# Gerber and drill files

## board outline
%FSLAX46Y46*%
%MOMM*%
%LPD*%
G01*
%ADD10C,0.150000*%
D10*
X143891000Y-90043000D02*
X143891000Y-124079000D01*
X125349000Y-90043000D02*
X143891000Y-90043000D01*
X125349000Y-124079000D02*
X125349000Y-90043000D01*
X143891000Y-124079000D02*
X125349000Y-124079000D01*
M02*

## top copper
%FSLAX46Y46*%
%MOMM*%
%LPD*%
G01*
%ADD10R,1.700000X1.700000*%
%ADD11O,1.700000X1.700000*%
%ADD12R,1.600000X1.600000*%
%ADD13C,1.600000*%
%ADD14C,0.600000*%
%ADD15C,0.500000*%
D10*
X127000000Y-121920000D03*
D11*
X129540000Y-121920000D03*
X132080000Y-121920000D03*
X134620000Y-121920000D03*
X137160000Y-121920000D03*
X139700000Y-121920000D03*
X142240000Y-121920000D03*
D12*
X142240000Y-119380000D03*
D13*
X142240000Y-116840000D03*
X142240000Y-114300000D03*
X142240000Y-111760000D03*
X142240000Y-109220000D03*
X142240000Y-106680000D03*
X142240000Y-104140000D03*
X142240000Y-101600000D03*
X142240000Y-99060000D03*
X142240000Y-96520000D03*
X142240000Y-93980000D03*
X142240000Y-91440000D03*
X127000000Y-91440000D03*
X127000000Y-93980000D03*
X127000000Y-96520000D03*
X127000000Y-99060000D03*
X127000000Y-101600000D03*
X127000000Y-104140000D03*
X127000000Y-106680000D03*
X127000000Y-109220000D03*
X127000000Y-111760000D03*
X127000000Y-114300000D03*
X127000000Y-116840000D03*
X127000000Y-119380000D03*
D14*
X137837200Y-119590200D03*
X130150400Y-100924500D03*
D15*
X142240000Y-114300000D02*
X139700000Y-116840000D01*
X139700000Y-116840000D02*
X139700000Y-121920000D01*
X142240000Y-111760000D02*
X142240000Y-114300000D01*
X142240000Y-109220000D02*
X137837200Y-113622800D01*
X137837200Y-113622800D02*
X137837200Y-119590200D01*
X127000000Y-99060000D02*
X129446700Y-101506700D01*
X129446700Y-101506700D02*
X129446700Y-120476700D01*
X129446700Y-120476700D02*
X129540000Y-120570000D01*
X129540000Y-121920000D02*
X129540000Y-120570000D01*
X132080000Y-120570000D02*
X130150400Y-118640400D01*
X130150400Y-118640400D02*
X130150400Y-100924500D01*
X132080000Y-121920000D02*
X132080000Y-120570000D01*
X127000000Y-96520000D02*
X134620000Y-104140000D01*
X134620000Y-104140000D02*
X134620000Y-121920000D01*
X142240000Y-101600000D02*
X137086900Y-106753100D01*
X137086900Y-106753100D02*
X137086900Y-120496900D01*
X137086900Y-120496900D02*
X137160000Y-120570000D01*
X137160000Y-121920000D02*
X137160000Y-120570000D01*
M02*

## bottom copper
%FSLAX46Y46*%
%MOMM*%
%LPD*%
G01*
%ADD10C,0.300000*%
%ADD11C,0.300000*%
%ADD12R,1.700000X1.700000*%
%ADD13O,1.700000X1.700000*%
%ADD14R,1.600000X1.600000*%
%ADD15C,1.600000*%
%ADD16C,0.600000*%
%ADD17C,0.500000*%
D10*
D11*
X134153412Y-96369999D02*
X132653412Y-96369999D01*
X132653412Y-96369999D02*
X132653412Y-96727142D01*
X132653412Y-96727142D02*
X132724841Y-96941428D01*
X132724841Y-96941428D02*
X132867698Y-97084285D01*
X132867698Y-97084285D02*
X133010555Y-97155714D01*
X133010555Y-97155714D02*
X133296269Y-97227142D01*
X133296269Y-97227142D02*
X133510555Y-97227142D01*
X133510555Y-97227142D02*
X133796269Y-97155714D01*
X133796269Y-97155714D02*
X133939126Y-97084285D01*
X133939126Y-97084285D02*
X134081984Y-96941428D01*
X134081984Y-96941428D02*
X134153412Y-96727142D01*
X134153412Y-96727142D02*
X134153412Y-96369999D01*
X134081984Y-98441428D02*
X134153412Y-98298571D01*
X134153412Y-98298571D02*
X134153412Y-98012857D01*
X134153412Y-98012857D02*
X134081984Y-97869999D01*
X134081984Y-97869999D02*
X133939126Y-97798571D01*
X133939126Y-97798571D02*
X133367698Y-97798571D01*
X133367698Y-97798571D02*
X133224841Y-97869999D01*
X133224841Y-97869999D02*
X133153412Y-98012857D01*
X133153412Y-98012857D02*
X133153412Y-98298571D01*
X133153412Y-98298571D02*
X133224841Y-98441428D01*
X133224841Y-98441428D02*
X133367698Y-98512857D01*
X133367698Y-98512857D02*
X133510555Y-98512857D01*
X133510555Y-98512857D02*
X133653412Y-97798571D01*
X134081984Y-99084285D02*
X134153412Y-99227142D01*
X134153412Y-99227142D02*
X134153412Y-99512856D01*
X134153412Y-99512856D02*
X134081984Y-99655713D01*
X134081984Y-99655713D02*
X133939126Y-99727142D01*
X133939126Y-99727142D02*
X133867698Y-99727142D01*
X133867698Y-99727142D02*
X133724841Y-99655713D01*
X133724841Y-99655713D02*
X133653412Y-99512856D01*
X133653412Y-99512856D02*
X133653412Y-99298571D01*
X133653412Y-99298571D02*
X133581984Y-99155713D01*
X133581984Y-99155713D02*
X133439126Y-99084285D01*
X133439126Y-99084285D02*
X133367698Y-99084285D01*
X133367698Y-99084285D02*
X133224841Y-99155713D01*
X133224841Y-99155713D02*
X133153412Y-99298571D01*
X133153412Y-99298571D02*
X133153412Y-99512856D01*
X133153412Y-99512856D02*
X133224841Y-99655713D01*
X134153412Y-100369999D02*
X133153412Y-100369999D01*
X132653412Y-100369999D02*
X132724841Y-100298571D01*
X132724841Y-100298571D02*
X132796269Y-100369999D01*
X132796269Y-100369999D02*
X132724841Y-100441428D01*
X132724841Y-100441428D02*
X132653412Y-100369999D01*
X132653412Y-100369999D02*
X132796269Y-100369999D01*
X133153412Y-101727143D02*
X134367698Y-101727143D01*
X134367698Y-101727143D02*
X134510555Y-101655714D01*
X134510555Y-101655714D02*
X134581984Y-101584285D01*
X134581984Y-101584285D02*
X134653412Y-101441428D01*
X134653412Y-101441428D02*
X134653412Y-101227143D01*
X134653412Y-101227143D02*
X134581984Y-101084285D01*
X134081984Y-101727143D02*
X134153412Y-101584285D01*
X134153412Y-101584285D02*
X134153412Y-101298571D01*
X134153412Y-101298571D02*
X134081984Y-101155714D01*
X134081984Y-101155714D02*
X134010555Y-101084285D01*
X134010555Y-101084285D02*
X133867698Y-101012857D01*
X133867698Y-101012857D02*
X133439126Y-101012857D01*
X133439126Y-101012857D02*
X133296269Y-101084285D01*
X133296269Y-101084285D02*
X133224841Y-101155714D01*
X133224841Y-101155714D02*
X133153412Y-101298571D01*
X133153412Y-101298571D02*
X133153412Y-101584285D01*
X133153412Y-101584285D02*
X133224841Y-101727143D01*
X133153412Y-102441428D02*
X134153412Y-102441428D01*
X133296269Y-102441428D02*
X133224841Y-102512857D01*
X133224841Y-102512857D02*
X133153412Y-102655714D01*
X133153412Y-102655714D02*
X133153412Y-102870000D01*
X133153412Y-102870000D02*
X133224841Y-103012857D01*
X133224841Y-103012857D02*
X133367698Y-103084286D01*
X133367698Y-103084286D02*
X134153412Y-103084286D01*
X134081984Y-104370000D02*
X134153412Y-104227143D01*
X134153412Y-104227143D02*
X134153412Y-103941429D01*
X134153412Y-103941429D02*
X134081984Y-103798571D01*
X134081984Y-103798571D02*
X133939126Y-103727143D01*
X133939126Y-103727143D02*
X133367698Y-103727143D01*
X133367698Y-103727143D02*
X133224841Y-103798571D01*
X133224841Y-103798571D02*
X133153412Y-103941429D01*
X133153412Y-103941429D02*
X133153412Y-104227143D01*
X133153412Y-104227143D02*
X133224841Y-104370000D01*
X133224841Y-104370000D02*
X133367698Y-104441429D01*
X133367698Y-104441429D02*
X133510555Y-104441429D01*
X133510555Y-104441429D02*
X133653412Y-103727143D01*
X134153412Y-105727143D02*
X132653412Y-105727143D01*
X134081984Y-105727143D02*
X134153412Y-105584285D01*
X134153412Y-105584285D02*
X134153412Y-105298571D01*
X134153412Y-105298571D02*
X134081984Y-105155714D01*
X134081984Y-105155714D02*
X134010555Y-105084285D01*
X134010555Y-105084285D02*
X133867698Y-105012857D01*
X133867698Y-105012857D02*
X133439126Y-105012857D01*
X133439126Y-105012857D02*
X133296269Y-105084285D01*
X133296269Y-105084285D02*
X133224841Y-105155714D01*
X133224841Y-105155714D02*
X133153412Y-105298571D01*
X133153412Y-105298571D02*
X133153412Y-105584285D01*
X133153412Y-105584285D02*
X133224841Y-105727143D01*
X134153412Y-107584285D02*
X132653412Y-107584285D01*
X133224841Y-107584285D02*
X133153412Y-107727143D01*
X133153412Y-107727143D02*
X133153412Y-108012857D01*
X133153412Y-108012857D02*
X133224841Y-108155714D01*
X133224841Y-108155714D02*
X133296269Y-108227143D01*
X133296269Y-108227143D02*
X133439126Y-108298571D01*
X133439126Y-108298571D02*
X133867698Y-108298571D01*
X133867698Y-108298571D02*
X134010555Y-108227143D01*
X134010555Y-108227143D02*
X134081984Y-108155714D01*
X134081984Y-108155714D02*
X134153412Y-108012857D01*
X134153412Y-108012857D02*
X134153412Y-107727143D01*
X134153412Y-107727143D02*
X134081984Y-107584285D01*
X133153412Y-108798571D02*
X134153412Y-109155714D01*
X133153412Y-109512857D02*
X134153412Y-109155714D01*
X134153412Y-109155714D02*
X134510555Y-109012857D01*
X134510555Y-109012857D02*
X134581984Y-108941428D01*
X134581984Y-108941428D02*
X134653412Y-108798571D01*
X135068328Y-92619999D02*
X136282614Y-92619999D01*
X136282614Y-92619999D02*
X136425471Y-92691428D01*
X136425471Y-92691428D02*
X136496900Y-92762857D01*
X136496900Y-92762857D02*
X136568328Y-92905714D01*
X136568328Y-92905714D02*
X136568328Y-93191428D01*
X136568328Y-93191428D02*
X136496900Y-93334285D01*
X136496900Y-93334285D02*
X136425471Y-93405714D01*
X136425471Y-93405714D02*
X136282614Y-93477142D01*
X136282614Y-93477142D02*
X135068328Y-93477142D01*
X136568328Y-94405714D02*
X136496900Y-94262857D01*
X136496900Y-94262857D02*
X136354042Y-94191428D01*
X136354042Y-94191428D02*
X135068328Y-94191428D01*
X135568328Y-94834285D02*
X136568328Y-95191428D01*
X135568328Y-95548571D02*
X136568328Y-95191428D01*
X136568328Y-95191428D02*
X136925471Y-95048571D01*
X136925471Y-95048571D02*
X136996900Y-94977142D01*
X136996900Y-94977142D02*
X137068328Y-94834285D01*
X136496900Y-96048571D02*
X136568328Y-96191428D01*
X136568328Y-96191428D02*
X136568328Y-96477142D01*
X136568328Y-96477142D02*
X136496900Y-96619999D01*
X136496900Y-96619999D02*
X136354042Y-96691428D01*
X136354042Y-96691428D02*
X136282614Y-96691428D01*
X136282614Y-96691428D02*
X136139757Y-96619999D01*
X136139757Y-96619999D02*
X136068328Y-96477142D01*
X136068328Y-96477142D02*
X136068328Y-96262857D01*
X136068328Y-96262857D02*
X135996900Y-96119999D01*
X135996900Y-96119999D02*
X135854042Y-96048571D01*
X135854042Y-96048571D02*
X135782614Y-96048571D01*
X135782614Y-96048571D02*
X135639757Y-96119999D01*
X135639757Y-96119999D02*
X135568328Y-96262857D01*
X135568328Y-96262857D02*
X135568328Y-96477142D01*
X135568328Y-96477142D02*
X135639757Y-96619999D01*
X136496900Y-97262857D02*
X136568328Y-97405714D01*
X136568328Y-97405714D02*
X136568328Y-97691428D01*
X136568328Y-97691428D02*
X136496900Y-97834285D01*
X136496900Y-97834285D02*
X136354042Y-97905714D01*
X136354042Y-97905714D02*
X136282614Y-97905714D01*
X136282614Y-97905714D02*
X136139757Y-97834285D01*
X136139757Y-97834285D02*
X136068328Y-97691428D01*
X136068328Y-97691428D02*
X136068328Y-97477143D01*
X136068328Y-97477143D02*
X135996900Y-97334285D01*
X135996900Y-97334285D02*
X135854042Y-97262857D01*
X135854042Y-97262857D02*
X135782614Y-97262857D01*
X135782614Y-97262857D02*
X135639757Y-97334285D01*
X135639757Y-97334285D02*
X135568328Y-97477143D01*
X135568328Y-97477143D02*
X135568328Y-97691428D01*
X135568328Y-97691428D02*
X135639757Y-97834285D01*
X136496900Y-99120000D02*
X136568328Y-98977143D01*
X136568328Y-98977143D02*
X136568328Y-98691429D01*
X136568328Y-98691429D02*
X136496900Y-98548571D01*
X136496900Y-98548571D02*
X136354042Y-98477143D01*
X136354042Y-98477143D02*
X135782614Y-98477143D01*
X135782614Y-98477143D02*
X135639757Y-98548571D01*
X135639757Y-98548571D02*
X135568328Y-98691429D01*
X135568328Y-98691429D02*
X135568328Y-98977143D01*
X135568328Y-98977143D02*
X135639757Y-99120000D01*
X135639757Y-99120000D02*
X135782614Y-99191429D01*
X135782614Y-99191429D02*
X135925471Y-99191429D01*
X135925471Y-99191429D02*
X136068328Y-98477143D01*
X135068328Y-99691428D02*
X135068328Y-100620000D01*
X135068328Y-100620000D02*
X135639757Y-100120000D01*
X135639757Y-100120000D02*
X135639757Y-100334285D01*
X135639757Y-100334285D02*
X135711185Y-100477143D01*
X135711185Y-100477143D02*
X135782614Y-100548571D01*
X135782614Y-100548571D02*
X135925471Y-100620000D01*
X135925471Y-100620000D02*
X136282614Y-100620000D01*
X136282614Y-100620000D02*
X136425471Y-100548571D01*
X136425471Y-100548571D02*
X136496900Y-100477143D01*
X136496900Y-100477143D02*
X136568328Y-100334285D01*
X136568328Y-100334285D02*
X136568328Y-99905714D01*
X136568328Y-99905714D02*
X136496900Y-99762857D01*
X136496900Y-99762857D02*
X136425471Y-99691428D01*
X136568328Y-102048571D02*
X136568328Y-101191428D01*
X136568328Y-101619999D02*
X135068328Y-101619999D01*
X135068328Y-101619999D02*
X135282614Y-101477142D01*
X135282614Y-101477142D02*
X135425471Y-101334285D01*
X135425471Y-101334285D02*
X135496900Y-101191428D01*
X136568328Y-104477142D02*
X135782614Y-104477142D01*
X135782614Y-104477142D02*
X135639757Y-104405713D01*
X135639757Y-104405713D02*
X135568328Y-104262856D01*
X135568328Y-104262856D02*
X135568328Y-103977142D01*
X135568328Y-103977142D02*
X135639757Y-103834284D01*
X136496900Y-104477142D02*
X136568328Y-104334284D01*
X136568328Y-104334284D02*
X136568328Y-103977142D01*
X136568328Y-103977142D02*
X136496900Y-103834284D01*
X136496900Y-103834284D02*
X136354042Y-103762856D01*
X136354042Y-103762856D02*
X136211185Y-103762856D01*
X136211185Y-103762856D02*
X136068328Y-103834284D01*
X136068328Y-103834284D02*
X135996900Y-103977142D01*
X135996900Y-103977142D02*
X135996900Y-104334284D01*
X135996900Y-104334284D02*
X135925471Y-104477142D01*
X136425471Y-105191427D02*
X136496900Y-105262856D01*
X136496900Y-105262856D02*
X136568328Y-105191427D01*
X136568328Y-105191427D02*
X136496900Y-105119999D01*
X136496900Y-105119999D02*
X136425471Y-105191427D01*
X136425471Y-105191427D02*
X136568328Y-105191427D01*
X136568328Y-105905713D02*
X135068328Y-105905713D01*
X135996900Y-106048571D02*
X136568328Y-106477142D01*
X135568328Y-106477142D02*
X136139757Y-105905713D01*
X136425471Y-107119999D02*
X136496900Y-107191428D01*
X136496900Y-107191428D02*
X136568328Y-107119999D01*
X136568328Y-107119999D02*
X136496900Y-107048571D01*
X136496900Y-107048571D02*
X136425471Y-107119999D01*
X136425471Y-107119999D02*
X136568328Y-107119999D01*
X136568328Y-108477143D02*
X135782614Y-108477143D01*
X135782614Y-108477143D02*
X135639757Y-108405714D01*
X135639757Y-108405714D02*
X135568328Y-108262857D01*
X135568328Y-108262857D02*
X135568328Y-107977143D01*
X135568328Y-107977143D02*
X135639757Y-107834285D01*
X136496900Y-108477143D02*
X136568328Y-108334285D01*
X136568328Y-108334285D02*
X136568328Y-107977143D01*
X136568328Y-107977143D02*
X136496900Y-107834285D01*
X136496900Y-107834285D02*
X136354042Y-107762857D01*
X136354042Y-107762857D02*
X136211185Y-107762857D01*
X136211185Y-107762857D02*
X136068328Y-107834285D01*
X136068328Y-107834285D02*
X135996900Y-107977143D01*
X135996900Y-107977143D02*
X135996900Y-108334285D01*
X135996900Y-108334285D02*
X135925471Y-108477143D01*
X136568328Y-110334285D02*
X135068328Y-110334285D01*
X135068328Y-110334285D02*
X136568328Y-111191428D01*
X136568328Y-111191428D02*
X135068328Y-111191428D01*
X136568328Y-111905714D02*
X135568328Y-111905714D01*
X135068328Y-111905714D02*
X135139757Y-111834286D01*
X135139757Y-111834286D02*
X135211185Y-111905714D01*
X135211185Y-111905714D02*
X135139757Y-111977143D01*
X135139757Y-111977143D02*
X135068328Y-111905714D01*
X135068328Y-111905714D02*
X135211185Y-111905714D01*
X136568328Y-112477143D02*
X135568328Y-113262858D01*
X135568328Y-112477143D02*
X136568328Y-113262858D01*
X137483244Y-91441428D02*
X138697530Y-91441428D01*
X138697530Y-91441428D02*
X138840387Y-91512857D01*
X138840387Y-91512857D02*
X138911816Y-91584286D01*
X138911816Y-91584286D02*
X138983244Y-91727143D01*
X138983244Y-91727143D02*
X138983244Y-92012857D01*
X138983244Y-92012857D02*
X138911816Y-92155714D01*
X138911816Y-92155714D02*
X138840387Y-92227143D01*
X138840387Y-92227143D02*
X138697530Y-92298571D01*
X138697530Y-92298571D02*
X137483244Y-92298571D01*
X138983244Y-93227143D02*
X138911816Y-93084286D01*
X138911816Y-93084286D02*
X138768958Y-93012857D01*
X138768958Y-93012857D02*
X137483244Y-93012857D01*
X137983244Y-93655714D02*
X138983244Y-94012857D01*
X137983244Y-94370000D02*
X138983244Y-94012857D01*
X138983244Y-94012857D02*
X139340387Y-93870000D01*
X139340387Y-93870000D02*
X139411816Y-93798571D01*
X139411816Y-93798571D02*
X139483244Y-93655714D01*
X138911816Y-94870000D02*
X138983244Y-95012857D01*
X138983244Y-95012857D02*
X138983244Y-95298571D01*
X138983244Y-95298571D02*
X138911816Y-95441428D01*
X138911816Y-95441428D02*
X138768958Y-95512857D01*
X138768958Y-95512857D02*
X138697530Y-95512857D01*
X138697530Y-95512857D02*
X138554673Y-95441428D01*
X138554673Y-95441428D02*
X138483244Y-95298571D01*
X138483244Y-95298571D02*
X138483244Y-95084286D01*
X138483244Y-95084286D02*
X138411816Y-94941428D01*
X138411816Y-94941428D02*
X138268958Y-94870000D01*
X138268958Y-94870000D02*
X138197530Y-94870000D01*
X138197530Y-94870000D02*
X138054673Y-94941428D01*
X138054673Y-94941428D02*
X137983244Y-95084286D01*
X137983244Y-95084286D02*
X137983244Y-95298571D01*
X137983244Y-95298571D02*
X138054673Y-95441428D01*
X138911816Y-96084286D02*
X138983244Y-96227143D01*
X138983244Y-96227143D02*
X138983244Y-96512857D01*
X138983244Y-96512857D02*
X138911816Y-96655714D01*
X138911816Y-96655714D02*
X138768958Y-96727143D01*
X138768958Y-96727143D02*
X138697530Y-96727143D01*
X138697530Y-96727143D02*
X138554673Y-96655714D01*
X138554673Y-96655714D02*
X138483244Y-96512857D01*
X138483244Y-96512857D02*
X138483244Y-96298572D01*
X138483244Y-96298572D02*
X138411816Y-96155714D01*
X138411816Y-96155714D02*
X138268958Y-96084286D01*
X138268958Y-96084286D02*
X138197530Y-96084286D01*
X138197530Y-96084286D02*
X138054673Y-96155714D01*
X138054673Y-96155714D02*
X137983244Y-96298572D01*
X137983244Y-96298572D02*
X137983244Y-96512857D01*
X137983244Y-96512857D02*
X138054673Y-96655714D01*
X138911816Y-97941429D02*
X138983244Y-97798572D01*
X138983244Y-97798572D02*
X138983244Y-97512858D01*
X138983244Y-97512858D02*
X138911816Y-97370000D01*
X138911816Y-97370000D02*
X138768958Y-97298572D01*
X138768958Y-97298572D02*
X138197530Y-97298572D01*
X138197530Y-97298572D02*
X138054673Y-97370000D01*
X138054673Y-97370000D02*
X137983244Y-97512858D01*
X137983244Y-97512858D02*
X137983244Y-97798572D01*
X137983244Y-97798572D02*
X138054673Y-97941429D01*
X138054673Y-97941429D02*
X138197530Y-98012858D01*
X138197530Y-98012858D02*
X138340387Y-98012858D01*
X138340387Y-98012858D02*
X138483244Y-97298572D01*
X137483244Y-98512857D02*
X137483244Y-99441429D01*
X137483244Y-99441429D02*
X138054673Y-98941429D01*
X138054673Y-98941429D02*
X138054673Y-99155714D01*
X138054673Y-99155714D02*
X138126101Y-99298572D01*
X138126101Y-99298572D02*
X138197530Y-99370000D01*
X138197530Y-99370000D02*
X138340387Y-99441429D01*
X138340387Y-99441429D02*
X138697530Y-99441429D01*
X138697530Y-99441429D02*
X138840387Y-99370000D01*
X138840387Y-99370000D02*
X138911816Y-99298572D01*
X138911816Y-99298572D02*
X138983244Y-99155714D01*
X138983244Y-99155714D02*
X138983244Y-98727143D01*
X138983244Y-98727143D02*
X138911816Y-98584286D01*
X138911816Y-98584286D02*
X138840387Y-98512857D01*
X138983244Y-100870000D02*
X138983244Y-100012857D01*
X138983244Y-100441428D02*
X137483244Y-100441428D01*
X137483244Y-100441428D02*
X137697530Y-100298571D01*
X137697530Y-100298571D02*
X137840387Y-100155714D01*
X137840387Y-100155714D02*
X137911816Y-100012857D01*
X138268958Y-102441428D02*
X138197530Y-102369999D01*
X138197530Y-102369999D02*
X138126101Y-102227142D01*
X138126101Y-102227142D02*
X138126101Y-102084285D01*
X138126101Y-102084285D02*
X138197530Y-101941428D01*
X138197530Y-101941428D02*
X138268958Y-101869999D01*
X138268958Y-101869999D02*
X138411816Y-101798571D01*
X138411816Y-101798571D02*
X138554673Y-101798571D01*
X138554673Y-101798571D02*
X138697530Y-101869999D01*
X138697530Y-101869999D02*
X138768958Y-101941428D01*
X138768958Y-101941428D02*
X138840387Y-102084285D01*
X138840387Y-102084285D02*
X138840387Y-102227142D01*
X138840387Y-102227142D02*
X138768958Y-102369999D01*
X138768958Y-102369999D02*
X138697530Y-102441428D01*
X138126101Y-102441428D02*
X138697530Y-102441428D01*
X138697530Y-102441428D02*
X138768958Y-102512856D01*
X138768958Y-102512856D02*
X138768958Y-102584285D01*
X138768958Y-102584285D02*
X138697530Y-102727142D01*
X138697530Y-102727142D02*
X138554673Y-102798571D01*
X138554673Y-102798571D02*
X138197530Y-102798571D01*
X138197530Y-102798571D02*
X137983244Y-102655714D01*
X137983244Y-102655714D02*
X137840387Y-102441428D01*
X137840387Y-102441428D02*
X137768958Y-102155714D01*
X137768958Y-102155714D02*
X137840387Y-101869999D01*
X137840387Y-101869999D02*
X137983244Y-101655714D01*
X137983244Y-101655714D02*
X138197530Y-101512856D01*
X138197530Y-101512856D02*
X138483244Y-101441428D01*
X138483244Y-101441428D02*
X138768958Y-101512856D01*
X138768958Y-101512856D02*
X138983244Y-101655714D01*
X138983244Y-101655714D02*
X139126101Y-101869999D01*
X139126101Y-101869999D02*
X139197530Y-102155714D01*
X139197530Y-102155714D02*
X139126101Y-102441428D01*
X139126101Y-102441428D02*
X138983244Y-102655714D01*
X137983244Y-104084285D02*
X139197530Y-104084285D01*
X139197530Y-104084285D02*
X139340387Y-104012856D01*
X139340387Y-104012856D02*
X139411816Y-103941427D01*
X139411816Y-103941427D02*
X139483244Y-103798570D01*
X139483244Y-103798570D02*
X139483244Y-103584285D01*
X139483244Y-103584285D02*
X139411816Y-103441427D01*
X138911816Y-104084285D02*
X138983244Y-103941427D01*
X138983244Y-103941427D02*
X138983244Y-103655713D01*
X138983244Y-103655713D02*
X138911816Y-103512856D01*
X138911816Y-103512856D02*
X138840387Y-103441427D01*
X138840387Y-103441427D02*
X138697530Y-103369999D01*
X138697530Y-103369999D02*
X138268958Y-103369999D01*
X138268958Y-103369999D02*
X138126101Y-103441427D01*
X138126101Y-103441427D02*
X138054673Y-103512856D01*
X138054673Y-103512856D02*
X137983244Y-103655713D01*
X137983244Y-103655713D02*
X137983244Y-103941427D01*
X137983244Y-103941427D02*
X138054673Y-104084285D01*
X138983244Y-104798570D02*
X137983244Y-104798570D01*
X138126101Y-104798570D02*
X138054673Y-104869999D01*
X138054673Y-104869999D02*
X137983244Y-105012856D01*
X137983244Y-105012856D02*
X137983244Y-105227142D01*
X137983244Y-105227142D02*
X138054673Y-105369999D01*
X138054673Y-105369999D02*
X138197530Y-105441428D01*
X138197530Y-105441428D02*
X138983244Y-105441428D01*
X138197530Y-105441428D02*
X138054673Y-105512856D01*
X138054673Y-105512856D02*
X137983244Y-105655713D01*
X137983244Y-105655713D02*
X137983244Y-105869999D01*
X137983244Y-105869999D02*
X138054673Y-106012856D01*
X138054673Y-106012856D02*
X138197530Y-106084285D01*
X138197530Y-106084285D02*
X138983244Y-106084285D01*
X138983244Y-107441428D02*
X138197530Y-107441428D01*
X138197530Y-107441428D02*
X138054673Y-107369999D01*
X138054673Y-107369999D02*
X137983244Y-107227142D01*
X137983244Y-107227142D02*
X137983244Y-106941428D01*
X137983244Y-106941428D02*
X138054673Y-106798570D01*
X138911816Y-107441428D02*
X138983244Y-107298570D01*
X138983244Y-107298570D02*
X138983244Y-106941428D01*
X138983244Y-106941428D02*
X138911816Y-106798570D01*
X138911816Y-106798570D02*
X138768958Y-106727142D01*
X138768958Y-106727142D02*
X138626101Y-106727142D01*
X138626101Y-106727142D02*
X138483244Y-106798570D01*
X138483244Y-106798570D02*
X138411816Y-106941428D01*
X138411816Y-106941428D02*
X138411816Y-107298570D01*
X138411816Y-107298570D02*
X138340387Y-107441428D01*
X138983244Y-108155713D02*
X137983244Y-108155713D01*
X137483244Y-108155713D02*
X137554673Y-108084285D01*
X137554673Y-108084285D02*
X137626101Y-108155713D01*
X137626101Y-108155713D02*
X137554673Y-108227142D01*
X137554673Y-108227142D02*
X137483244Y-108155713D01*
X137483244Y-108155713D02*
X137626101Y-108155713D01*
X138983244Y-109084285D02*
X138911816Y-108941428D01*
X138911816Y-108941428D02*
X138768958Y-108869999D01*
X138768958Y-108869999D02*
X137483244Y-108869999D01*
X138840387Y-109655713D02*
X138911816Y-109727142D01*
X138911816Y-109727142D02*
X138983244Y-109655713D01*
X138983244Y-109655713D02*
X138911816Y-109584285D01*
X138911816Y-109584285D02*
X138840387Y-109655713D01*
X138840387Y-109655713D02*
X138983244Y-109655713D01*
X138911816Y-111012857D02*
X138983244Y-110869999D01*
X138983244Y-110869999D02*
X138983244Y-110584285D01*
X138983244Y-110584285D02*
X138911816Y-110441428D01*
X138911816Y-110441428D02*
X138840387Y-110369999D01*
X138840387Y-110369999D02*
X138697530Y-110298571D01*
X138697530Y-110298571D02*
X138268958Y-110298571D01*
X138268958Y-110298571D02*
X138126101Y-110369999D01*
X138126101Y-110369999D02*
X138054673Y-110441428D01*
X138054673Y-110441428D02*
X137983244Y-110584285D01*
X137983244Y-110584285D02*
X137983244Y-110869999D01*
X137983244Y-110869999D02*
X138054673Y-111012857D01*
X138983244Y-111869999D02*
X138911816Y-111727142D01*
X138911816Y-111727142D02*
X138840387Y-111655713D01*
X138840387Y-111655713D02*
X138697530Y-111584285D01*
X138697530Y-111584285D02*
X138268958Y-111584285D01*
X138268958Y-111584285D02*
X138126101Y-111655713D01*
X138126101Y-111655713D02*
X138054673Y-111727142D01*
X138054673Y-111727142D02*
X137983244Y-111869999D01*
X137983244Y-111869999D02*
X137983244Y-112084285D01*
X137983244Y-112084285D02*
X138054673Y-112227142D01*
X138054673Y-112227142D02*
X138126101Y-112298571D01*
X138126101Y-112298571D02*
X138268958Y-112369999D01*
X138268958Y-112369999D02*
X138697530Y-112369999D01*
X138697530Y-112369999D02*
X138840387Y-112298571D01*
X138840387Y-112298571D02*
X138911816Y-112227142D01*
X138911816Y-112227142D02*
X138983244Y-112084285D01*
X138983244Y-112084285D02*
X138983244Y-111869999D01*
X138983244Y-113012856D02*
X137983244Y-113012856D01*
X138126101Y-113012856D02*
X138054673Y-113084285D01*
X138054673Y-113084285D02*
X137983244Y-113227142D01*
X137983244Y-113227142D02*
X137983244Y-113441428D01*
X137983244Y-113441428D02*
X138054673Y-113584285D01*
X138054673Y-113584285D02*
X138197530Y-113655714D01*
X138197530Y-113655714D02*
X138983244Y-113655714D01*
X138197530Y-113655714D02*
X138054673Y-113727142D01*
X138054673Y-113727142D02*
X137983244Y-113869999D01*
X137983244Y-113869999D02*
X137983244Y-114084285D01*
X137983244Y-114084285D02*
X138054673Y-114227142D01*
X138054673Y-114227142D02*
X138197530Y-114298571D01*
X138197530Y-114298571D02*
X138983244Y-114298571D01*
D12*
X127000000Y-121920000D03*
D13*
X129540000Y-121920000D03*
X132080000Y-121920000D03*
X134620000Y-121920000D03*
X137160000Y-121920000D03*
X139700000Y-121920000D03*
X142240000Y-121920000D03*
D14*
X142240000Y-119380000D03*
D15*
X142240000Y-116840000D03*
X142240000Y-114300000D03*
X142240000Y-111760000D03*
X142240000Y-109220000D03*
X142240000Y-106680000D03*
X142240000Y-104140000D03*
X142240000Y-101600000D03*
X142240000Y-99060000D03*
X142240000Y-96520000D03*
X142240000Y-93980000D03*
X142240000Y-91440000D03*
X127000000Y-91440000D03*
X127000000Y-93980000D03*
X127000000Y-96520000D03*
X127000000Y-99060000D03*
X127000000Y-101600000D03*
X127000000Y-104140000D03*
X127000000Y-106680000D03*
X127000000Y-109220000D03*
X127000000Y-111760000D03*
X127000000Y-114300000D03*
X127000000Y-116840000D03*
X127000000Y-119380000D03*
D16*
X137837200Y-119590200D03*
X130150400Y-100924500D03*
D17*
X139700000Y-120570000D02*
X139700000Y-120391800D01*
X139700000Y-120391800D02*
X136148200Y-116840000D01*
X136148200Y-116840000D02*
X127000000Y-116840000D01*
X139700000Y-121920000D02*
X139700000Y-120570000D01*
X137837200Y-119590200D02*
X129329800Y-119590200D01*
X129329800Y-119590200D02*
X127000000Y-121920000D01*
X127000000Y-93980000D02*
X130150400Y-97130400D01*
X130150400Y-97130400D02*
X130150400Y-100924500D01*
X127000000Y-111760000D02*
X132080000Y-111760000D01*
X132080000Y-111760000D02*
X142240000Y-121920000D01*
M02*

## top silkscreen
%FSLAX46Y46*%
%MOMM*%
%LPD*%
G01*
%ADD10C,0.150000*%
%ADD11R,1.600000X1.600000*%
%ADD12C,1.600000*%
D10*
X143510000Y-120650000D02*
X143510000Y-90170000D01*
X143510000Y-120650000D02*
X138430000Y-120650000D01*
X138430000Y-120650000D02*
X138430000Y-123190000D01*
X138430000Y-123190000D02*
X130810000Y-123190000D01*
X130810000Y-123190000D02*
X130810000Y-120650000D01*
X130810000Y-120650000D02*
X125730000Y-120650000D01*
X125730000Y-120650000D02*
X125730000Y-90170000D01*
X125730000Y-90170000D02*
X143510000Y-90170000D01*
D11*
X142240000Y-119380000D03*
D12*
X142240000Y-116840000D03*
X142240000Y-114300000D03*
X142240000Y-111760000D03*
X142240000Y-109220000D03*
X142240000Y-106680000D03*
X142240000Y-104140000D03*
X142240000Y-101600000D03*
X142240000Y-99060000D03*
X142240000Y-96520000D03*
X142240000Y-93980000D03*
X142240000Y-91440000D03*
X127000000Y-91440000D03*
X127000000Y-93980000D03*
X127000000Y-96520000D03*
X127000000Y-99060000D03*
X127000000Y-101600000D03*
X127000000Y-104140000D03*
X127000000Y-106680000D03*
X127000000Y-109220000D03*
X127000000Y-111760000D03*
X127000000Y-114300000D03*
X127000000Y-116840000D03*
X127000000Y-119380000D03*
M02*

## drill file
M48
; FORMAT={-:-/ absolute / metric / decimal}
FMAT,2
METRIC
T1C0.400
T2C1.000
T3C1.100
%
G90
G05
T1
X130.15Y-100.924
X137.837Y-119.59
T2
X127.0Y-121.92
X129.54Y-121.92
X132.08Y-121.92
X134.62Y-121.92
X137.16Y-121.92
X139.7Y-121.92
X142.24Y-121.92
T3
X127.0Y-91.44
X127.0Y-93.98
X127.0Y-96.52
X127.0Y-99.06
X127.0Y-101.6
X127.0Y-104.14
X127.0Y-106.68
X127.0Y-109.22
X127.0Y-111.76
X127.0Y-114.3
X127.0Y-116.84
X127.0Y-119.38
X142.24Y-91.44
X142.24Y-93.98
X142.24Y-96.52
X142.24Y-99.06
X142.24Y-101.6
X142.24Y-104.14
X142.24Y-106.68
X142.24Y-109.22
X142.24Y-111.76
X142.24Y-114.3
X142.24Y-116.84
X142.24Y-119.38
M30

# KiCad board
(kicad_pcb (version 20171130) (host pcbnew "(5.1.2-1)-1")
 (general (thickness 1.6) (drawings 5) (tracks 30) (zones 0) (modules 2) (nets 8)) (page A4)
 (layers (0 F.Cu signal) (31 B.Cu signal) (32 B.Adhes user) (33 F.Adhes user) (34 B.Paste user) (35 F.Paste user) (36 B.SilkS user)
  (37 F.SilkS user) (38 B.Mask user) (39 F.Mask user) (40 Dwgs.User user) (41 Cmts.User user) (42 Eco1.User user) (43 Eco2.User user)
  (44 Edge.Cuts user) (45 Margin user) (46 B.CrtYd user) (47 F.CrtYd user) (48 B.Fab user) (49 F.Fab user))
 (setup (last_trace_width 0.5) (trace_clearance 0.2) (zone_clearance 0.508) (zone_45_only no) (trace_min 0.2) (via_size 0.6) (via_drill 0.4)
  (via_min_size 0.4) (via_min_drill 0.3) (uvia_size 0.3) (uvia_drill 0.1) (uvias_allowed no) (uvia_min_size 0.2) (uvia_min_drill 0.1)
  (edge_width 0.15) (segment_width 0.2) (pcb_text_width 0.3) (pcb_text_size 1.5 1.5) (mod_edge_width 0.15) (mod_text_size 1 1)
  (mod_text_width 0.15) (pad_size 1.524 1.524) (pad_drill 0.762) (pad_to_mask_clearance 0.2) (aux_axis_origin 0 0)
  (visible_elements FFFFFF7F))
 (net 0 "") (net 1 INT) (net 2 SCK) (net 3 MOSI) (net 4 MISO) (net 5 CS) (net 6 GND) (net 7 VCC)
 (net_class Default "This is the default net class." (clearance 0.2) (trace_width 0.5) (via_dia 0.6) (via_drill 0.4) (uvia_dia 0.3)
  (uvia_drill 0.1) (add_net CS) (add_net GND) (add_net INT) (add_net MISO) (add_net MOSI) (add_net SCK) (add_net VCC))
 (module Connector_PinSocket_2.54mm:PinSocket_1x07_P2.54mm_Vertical (layer B.Cu) (at 127 121.92 270)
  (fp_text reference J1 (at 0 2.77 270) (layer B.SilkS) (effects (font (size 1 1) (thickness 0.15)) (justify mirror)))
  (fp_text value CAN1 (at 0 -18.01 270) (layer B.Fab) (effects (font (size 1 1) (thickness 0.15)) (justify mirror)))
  (pad 1 thru_hole rect (at 0 0 270) (size 1.7 1.7) (drill 1) (layers *.Cu *.Mask) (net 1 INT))
  (pad 2 thru_hole oval (at 0 -2.54 270) (size 1.7 1.7) (drill 1) (layers *.Cu *.Mask) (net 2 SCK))
  (pad 3 thru_hole oval (at 0 -5.08 270) (size 1.7 1.7) (drill 1) (layers *.Cu *.Mask) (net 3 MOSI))
  (pad 4 thru_hole oval (at 0 -7.62 270) (size 1.7 1.7) (drill 1) (layers *.Cu *.Mask) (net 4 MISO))
  (pad 5 thru_hole oval (at 0 -10.16 270) (size 1.7 1.7) (drill 1) (layers *.Cu *.Mask) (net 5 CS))
  (pad 6 thru_hole oval (at 0 -12.7 270) (size 1.7 1.7) (drill 1) (layers *.Cu *.Mask) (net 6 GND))
  (pad 7 thru_hole oval (at 0 -15.24 270) (size 1.7 1.7) (drill 1) (layers *.Cu *.Mask) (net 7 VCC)))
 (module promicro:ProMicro (layer F.Cu) (at 134.62 105.41 90)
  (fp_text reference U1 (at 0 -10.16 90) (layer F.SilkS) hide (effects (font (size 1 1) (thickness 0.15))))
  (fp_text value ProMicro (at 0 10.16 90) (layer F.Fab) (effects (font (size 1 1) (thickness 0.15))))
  (fp_line (start -15.24 8.89) (end 15.24 8.89) (layer F.SilkS) (width 0.15))
  (fp_line (start -15.24 8.89) (end -15.24 3.81) (layer F.SilkS) (width 0.15))
  (fp_line (start -15.24 3.81) (end -17.78 3.81) (layer F.SilkS) (width 0.15))
  (fp_line (start -17.78 3.81) (end -17.78 -3.81) (layer F.SilkS) (width 0.15))
  (fp_line (start -17.78 -3.81) (end -15.24 -3.81) (layer F.SilkS) (width 0.15))
  (fp_line (start -15.24 -3.81) (end -15.24 -8.89) (layer F.SilkS) (width 0.15))
  (fp_line (start -15.24 -8.89) (end 15.24 -8.89) (layer F.SilkS) (width 0.15))
  (fp_line (start 15.24 -8.89) (end 15.24 8.89) (layer F.SilkS) (width 0.15))
  (pad 1 thru_hole rect (at -13.97 7.62 90) (size 1.6 1.6) (drill 1.1) (layers *.Cu *.Mask F.SilkS))
  (pad 2 thru_hole circle (at -11.43 7.62 90) (size 1.6 1.6) (drill 1.1) (layers *.Cu *.Mask F.SilkS))
  (pad 3 thru_hole circle (at -8.89 7.62 90) (size 1.6 1.6) (drill 1.1) (layers *.Cu *.Mask F.SilkS) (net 6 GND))
  (pad 4 thru_hole circle (at -6.35 7.62 90) (size 1.6 1.6) (drill 1.1) (layers *.Cu *.Mask F.SilkS) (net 6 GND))
  (pad 5 thru_hole circle (at -3.81 7.62 90) (size 1.6 1.6) (drill 1.1) (layers *.Cu *.Mask F.SilkS) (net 1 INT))
  (pad 6 thru_hole circle (at -1.27 7.62 90) (size 1.6 1.6) (drill 1.1) (layers *.Cu *.Mask F.SilkS))
  (pad 7 thru_hole circle (at 1.27 7.62 90) (size 1.6 1.6) (drill 1.1) (layers *.Cu *.Mask F.SilkS))
  (pad 8 thru_hole circle (at 3.81 7.62 90) (size 1.6 1.6) (drill 1.1) (layers *.Cu *.Mask F.SilkS) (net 5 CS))
  (pad 9 thru_hole circle (at 6.35 7.62 90) (size 1.6 1.6) (drill 1.1) (layers *.Cu *.Mask F.SilkS))
  (pad 10 thru_hole circle (at 8.89 7.62 90) (size 1.6 1.6) (drill 1.1) (layers *.Cu *.Mask F.SilkS))
  (pad 11 thru_hole circle (at 11.43 7.62 90) (size 1.6 1.6) (drill 1.1) (layers *.Cu *.Mask F.SilkS))
  (pad 12 thru_hole circle (at 13.97 7.62 90) (size 1.6 1.6) (drill 1.1) (layers *.Cu *.Mask F.SilkS))
  (pad 13 thru_hole circle (at 13.97 -7.62 90) (size 1.6 1.6) (drill 1.1) (layers *.Cu *.Mask F.SilkS))
  (pad 14 thru_hole circle (at 11.43 -7.62 90) (size 1.6 1.6) (drill 1.1) (layers *.Cu *.Mask F.SilkS) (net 3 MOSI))
  (pad 15 thru_hole circle (at 8.89 -7.62 90) (size 1.6 1.6) (drill 1.1) (layers *.Cu *.Mask F.SilkS) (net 4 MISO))
  (pad 16 thru_hole circle (at 6.35 -7.62 90) (size 1.6 1.6) (drill 1.1) (layers *.Cu *.Mask F.SilkS) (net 2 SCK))
  (pad 17 thru_hole circle (at 3.81 -7.62 90) (size 1.6 1.6) (drill 1.1) (layers *.Cu *.Mask F.SilkS))
  (pad 18 thru_hole circle (at 1.27 -7.62 90) (size 1.6 1.6) (drill 1.1) (layers *.Cu *.Mask F.SilkS))
  (pad 19 thru_hole circle (at -1.27 -7.62 90) (size 1.6 1.6) (drill 1.1) (layers *.Cu *.Mask F.SilkS))
  (pad 20 thru_hole circle (at -3.81 -7.62 90) (size 1.6 1.6) (drill 1.1) (layers *.Cu *.Mask F.SilkS))
  (pad 21 thru_hole circle (at -6.35 -7.62 90) (size 1.6 1.6) (drill 1.1) (layers *.Cu *.Mask F.SilkS) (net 7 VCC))
  (pad 22 thru_hole circle (at -8.89 -7.62 90) (size 1.6 1.6) (drill 1.1) (layers *.Cu *.Mask F.SilkS))
  (pad 23 thru_hole circle (at -11.43 -7.62 90) (size 1.6 1.6) (drill 1.1) (layers *.Cu *.Mask F.SilkS) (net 6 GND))
  (pad 24 thru_hole circle (at -13.97 -7.62 90) (size 1.6 1.6) (drill 1.1) (layers *.Cu *.Mask F.SilkS)))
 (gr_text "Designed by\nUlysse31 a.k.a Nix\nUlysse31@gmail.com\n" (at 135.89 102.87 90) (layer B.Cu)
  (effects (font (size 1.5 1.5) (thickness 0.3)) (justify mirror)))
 (gr_line (start 143.891 90.043) (end 143.891 124.079) (angle 90) (layer Edge.Cuts) (width 0.15))
 (gr_line (start 125.349 90.043) (end 143.891 90.043) (angle 90) (layer Edge.Cuts) (width 0.15))
 (gr_line (start 125.349 124.079) (end 125.349 90.043) (angle 90) (layer Edge.Cuts) (width 0.15))
 (gr_line (start 143.891 124.079) (end 125.349 124.079) (angle 90) (layer Edge.Cuts) (width 0.15))
 (segment (start 139.7 120.57) (end 139.7 120.3918) (width 0.5) (layer B.Cu) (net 6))
 (segment (start 139.7 120.3918) (end 136.1482 116.84) (width 0.5) (layer B.Cu) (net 6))
 (segment (start 136.1482 116.84) (end 127 116.84) (width 0.5) (layer B.Cu) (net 6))
 (segment (start 142.24 114.3) (end 139.7 116.84) (width 0.5) (layer F.Cu) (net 6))
 (segment (start 139.7 116.84) (end 139.7 121.92) (width 0.5) (layer F.Cu) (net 6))
 (segment (start 142.24 111.76) (end 142.24 114.3) (width 0.5) (layer F.Cu) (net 6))
 (segment (start 139.7 121.92) (end 139.7 120.57) (width 0.5) (layer B.Cu) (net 6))
 (segment (start 137.8372 119.5902) (end 129.3298 119.5902) (width 0.5) (layer B.Cu) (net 1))
 (segment (start 129.3298 119.5902) (end 127 121.92) (width 0.5) (layer B.Cu) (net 1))
 (segment (start 142.24 109.22) (end 137.8372 113.6228) (width 0.5) (layer F.Cu) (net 1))
 (segment (start 137.8372 113.6228) (end 137.8372 119.5902) (width 0.5) (layer F.Cu) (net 1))
 (via (at 137.8372 119.5902) (size 0.6) (layers F.Cu B.Cu) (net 1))
 (segment (start 127 99.06) (end 129.4467 101.5067) (width 0.5) (layer F.Cu) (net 2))
 (segment (start 129.4467 101.5067) (end 129.4467 120.4767) (width 0.5) (layer F.Cu) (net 2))
 (segment (start 129.4467 120.4767) (end 129.54 120.57) (width 0.5) (layer F.Cu) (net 2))
 (segment (start 129.54 121.92) (end 129.54 120.57) (width 0.5) (layer F.Cu) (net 2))
 (segment (start 132.08 120.57) (end 130.1504 118.6404) (width 0.5) (layer F.Cu) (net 3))
 (segment (start 130.1504 118.6404) (end 130.1504 100.9245) (width 0.5) (layer F.Cu) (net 3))
 (segment (start 127 93.98) (end 130.1504 97.1304) (width 0.5) (layer B.Cu) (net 3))
 (segment (start 130.1504 97.1304) (end 130.1504 100.9245) (width 0.5) (layer B.Cu) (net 3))
 (segment (start 132.08 121.92) (end 132.08 120.57) (width 0.5) (layer F.Cu) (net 3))
 (via (at 130.1504 100.9245) (size 0.6) (layers F.Cu B.Cu) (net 3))
 (segment (start 127 96.52) (end 134.62 104.14) (width 0.5) (layer F.Cu) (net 4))
 (segment (start 134.62 104.14) (end 134.62 121.92) (width 0.5) (layer F.Cu) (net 4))
 (segment (start 142.24 101.6) (end 137.0869 106.7531) (width 0.5) (layer F.Cu) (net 5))
 (segment (start 137.0869 106.7531) (end 137.0869 120.4969) (width 0.5) (layer F.Cu) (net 5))
 (segment (start 137.0869 120.4969) (end 137.16 120.57) (width 0.5) (layer F.Cu) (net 5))
 (segment (start 137.16 121.92) (end 137.16 120.57) (width 0.5) (layer F.Cu) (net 5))
 (segment (start 127 111.76) (end 132.08 111.76) (width 0.5) (layer B.Cu) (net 7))
 (segment (start 132.08 111.76) (end 142.24 121.92) (width 0.5) (layer B.Cu) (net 7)))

